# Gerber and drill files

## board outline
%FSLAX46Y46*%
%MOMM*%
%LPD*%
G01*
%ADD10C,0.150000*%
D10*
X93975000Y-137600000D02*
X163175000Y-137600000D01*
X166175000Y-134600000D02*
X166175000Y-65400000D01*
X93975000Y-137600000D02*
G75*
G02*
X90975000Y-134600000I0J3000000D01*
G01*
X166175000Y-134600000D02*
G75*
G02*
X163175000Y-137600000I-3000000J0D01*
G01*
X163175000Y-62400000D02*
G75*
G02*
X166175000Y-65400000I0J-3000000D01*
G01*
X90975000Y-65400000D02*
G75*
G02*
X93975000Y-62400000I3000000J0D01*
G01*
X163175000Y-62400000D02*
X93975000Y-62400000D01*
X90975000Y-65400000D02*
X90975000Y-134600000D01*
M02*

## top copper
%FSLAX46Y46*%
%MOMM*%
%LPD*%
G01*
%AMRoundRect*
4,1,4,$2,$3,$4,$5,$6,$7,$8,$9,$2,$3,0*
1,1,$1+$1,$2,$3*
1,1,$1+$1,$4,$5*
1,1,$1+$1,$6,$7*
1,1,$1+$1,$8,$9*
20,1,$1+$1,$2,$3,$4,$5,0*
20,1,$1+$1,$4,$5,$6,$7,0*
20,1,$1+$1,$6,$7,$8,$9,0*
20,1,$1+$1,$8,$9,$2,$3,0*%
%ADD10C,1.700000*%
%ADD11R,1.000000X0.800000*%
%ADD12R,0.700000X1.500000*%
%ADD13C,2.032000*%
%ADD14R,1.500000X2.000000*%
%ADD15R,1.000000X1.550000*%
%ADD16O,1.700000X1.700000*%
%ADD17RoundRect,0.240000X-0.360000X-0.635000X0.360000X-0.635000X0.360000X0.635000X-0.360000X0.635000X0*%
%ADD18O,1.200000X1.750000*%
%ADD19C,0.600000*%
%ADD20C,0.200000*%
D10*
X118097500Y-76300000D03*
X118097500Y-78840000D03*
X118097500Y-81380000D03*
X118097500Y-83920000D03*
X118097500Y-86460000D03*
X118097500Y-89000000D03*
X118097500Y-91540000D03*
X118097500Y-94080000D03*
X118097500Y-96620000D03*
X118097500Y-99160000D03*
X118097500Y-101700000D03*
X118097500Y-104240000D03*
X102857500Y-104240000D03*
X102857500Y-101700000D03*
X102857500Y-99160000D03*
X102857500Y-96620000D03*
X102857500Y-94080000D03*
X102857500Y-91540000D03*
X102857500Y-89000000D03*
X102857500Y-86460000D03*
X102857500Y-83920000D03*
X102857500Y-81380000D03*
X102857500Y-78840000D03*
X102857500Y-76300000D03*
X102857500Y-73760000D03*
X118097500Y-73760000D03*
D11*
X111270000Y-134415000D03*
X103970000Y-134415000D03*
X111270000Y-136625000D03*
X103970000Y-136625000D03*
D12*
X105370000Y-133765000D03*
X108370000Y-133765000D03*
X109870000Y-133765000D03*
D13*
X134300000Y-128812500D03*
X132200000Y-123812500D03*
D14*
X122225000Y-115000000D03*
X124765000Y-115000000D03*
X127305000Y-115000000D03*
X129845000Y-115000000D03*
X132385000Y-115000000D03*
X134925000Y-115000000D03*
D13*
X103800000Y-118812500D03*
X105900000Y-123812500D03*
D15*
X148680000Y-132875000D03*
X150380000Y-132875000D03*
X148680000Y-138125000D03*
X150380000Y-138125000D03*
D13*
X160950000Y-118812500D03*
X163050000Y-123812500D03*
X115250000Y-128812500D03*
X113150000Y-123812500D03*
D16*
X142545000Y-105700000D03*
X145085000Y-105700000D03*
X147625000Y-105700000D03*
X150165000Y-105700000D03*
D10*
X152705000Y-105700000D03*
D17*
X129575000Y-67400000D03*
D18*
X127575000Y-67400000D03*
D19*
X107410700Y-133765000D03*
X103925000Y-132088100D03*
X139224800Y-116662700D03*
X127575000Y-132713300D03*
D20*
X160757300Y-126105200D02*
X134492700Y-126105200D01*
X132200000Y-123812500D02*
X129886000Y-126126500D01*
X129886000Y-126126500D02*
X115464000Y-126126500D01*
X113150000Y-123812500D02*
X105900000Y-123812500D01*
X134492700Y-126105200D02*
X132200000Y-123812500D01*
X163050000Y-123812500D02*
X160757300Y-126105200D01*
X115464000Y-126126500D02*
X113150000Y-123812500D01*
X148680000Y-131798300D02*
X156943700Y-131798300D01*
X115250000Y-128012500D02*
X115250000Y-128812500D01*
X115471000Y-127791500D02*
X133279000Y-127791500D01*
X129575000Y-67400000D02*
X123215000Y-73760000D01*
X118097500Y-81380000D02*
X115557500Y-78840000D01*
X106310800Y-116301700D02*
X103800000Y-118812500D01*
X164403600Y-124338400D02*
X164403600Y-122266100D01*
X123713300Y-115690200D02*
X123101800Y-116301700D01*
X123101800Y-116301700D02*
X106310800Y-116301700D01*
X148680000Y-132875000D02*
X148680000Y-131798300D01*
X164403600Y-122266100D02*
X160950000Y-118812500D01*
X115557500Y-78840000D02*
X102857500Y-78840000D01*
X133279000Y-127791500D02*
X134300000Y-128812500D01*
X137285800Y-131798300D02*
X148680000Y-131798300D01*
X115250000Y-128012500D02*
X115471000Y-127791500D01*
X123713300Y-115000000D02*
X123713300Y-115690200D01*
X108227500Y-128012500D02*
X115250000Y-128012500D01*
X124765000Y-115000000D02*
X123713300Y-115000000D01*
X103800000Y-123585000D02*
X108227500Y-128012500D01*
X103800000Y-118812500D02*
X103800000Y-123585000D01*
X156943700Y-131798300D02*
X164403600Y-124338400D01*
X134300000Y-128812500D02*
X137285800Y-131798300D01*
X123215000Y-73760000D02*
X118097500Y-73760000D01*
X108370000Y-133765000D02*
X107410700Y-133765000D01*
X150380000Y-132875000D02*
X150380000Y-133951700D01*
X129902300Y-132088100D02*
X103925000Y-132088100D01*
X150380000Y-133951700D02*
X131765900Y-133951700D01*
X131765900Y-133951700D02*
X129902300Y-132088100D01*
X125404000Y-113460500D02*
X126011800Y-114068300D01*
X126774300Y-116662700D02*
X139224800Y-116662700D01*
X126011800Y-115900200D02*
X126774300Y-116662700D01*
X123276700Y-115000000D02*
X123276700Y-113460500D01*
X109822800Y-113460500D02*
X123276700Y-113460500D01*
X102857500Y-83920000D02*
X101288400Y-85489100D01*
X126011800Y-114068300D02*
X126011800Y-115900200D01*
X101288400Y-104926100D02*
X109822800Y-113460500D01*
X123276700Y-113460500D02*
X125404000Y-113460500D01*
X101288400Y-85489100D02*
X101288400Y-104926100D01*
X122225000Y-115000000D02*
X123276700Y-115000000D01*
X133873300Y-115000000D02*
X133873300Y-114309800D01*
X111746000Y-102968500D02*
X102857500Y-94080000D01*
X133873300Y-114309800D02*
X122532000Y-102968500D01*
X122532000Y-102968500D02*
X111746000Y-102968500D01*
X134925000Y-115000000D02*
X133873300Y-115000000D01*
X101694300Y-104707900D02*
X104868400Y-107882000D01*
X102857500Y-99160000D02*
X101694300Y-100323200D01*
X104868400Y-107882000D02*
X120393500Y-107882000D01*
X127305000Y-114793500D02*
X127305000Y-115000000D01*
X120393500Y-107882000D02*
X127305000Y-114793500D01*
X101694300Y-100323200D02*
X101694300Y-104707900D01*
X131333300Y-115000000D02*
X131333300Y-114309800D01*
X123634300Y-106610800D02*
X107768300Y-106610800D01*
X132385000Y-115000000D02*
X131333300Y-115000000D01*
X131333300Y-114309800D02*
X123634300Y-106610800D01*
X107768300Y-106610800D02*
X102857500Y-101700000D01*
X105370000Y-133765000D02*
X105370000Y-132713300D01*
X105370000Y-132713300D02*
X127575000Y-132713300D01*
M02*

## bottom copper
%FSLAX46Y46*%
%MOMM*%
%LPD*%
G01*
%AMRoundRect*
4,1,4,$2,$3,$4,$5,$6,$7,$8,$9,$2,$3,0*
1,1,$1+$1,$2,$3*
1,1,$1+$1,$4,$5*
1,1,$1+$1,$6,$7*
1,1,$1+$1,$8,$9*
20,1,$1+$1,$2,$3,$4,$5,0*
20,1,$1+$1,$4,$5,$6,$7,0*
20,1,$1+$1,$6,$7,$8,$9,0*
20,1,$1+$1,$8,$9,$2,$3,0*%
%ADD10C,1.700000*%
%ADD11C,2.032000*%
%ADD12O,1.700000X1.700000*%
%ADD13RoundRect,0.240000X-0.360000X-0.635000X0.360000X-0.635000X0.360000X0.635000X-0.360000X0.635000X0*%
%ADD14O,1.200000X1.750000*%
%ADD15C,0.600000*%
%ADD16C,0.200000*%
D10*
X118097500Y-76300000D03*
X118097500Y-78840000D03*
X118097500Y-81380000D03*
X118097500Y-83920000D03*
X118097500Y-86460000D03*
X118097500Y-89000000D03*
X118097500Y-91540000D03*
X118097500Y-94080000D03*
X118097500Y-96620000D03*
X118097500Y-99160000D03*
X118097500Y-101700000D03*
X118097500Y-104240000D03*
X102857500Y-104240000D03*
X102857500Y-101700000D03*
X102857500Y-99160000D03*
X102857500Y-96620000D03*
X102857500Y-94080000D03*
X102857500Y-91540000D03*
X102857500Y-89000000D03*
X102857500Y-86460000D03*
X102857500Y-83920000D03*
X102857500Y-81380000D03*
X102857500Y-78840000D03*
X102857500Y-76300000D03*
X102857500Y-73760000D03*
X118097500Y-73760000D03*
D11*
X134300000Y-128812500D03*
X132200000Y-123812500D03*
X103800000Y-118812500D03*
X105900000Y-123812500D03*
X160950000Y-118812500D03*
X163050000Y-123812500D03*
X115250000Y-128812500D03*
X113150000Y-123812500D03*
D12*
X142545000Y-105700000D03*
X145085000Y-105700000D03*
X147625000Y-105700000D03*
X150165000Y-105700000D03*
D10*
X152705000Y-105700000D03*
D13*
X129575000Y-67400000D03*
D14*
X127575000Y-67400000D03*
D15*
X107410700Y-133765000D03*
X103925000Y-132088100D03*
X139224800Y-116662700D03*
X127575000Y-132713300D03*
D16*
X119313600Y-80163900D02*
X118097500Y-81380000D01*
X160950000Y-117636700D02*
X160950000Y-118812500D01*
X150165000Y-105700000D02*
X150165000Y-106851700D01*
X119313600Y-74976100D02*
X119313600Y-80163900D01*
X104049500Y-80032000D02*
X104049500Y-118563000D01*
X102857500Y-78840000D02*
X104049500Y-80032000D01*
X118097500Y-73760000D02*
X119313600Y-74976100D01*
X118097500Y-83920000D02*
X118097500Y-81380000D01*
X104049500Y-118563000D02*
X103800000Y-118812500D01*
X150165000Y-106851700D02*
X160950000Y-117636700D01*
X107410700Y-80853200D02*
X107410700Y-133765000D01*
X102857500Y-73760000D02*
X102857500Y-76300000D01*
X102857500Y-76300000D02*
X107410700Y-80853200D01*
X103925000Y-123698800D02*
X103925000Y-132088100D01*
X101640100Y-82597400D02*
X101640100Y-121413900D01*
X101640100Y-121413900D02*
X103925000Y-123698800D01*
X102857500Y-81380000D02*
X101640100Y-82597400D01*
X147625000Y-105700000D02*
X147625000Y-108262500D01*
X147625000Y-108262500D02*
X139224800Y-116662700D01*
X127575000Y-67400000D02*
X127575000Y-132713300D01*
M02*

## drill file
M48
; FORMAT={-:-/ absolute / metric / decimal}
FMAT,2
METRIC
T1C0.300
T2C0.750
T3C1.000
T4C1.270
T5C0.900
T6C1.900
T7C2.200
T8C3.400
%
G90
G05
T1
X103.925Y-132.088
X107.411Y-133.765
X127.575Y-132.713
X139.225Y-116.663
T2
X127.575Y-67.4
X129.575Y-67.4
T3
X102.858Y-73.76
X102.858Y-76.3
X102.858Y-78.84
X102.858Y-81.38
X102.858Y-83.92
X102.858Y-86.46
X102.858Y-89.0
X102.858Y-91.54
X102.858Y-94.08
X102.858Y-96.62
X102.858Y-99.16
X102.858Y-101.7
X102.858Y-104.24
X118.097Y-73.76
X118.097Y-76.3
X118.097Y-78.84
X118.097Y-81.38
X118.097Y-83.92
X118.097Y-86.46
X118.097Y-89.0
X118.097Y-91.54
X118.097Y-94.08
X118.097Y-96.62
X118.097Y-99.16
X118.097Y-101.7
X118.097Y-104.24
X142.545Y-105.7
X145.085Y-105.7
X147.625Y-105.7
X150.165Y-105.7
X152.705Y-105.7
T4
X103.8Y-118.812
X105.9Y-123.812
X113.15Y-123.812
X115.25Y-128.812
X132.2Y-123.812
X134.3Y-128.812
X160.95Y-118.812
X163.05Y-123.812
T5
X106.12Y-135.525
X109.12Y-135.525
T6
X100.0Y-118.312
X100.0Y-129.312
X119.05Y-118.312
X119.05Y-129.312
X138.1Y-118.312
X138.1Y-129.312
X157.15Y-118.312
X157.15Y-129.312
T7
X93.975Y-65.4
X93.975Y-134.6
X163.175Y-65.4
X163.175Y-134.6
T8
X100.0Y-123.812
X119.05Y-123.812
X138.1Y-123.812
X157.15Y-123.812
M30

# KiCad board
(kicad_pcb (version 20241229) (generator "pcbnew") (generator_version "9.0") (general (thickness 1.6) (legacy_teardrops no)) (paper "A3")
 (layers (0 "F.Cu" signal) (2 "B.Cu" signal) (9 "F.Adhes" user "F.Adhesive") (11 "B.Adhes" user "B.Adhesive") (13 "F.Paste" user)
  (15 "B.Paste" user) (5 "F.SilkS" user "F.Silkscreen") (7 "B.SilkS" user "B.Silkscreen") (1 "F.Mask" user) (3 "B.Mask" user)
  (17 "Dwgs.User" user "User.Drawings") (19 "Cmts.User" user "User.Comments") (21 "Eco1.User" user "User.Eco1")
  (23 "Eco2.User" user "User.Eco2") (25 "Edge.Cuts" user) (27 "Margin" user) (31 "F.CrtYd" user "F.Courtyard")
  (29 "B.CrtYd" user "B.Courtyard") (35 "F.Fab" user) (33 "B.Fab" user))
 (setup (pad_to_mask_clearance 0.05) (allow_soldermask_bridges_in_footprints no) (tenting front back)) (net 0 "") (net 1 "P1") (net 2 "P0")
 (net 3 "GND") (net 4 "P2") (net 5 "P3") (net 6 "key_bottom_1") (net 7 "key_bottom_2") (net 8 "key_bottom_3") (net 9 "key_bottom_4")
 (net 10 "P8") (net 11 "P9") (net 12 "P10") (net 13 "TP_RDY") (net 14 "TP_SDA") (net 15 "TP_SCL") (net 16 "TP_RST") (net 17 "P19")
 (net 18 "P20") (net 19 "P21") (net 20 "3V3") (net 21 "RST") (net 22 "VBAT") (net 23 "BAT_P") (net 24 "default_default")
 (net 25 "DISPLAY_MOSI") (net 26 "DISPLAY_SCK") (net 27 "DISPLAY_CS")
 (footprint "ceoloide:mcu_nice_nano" (layer "F.Cu") (at 110.4775 89)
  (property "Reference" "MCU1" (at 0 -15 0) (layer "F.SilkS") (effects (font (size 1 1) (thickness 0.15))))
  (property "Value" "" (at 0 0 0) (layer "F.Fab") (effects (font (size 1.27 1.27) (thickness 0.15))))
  (pad "1" thru_hole circle (at 7.62 -12.7) (size 1.7 1.7) (drill 1) (layers "*.Cu" "*.Mask") (remove_unused_layers no) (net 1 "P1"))
  (pad "2" thru_hole circle (at 7.62 -10.16) (size 1.7 1.7) (drill 1) (layers "*.Cu" "*.Mask") (remove_unused_layers no) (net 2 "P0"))
  (pad "3" thru_hole circle (at 7.62 -7.62) (size 1.7 1.7) (drill 1) (layers "*.Cu" "*.Mask") (remove_unused_layers no) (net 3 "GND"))
  (pad "4" thru_hole circle (at 7.62 -5.08) (size 1.7 1.7) (drill 1) (layers "*.Cu" "*.Mask") (remove_unused_layers no) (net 3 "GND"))
  (pad "5" thru_hole circle (at 7.62 -2.54) (size 1.7 1.7) (drill 1) (layers "*.Cu" "*.Mask") (remove_unused_layers no) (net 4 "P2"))
  (pad "6" thru_hole circle (at 7.62 0) (size 1.7 1.7) (drill 1) (layers "*.Cu" "*.Mask") (remove_unused_layers no) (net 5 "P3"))
  (pad "7" thru_hole circle (at 7.62 2.54) (size 1.7 1.7) (drill 1) (layers "*.Cu" "*.Mask") (remove_unused_layers no)
   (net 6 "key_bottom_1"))
  (pad "8" thru_hole circle (at 7.62 5.08) (size 1.7 1.7) (drill 1) (layers "*.Cu" "*.Mask") (remove_unused_layers no)
   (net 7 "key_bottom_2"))
  (pad "9" thru_hole circle (at 7.62 7.62) (size 1.7 1.7) (drill 1) (layers "*.Cu" "*.Mask") (remove_unused_layers no)
   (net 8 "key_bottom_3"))
  (pad "10" thru_hole circle (at 7.62 10.16) (size 1.7 1.7) (drill 1) (layers "*.Cu" "*.Mask") (remove_unused_layers no)
   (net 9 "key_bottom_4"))
  (pad "11" thru_hole circle (at 7.62 12.7) (size 1.7 1.7) (drill 1) (layers "*.Cu" "*.Mask") (remove_unused_layers no) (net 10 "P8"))
  (pad "12" thru_hole circle (at 7.62 15.24) (size 1.7 1.7) (drill 1) (layers "*.Cu" "*.Mask") (remove_unused_layers no) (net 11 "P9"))
  (pad "13" thru_hole circle (at -7.62 15.24) (size 1.7 1.7) (drill 1) (layers "*.Cu" "*.Mask") (remove_unused_layers no) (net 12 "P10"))
  (pad "14" thru_hole circle (at -7.62 12.7) (size 1.7 1.7) (drill 1) (layers "*.Cu" "*.Mask") (remove_unused_layers no) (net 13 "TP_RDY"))
  (pad "15" thru_hole circle (at -7.62 10.16) (size 1.7 1.7) (drill 1) (layers "*.Cu" "*.Mask") (remove_unused_layers no) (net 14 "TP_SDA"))
  (pad "16" thru_hole circle (at -7.62 7.62) (size 1.7 1.7) (drill 1) (layers "*.Cu" "*.Mask") (remove_unused_layers no) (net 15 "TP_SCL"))
  (pad "17" thru_hole circle (at -7.62 5.08) (size 1.7 1.7) (drill 1) (layers "*.Cu" "*.Mask") (remove_unused_layers no) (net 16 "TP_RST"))
  (pad "18" thru_hole circle (at -7.62 2.54) (size 1.7 1.7) (drill 1) (layers "*.Cu" "*.Mask") (remove_unused_layers no) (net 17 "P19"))
  (pad "19" thru_hole circle (at -7.62 0) (size 1.7 1.7) (drill 1) (layers "*.Cu" "*.Mask") (remove_unused_layers no) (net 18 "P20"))
  (pad "20" thru_hole circle (at -7.62 -2.54) (size 1.7 1.7) (drill 1) (layers "*.Cu" "*.Mask") (remove_unused_layers no) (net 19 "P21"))
  (pad "21" thru_hole circle (at -7.62 -5.08) (size 1.7 1.7) (drill 1) (layers "*.Cu" "*.Mask") (remove_unused_layers no) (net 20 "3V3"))
  (pad "22" thru_hole circle (at -7.62 -7.62) (size 1.7 1.7) (drill 1) (layers "*.Cu" "*.Mask") (remove_unused_layers no) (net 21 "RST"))
  (pad "23" thru_hole circle (at -7.62 -10.16) (size 1.7 1.7) (drill 1) (layers "*.Cu" "*.Mask") (remove_unused_layers no) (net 3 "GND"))
  (pad "24" thru_hole circle (at -7.62 -12.7) (size 1.7 1.7) (drill 1) (layers "*.Cu" "*.Mask") (remove_unused_layers no) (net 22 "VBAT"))
  (pad "25" thru_hole circle (at -7.62 -15.24) (size 1.7 1.7) (drill 1) (layers "*.Cu" "*.Mask") (remove_unused_layers no) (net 22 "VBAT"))
  (pad "26" thru_hole circle (at 7.62 -15.24) (size 1.7 1.7) (drill 1) (layers "*.Cu" "*.Mask") (remove_unused_layers no) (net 3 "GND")))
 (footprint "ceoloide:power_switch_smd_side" (layer "F.Cu") (at 107.62 135.5 -90)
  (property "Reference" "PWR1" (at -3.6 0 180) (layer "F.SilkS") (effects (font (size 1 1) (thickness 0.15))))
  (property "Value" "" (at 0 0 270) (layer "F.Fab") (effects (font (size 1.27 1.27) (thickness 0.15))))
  (pad "" smd rect (at -1.085 -3.65) (size 1 0.8) (layers "F.Cu" "F.Mask" "F.Paste"))
  (pad "" smd rect (at -1.085 3.65) (size 1 0.8) (layers "F.Cu" "F.Mask" "F.Paste"))
  (pad "" np_thru_hole circle (at 0.025 -1.5) (size 0.9 0.9) (drill 0.9) (layers "*.Cu" "*.Mask"))
  (pad "" np_thru_hole circle (at 0.025 1.5) (size 0.9 0.9) (drill 0.9) (layers "*.Cu" "*.Mask"))
  (pad "" smd rect (at 1.125 -3.65) (size 1 0.8) (layers "F.Cu" "F.Mask" "F.Paste"))
  (pad "" smd rect (at 1.125 3.65) (size 1 0.8) (layers "F.Cu" "F.Mask" "F.Paste"))
  (pad "1" smd rect (at -1.735 2.25) (size 0.7 1.5) (layers "F.Cu" "F.Mask" "F.Paste") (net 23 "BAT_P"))
  (pad "2" smd rect (at -1.735 -0.75) (size 0.7 1.5) (layers "F.Cu" "F.Mask" "F.Paste") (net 22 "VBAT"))
  (pad "3" smd rect (at -1.735 -2.25) (size 0.7 1.5) (layers "F.Cu" "F.Mask" "F.Paste")))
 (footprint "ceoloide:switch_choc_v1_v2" (layer "F.Cu") (at 138.1 123.8125 90)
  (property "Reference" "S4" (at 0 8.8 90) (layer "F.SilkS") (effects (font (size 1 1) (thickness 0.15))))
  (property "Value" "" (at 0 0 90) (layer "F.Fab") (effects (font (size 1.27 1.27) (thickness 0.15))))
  (pad "" np_thru_hole circle (at -5.5 0 90) (size 1.9 1.9) (drill 1.9) (layers "*.Cu" "*.Mask"))
  (pad "" np_thru_hole circle (at 0 0 90) (size 3.4 3.4) (drill 3.4) (layers "*.Cu" "*.Mask"))
  (pad "" np_thru_hole circle (at 5.5 0 90) (size 1.9 1.9) (drill 1.9) (layers "*.Cu" "*.Mask"))
  (pad "1" thru_hole circle (at -5 -3.8 285) (size 2.032 2.032) (drill 1.27) (layers "*.Cu" "*.Mask") (remove_unused_layers no)
   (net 3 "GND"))
  (pad "2" thru_hole circle (at 0 -5.9 285) (size 2.032 2.032) (drill 1.27) (layers "*.Cu" "*.Mask") (remove_unused_layers no)
   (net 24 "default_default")))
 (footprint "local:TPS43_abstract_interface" (layer "F.Cu") (at 128.575 91)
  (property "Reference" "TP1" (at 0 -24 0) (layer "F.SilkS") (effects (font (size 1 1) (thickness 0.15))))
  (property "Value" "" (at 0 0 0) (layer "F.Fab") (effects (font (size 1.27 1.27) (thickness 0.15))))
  (pad "1" smd rect (at -6.35 24) (size 1.5 2) (layers "F.Cu" "F.Mask" "F.Paste") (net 20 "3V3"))
  (pad "2" smd rect (at -3.81 24) (size 1.5 2) (layers "F.Cu" "F.Mask" "F.Paste") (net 3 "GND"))
  (pad "3" smd rect (at -1.27 24) (size 1.5 2) (layers "F.Cu" "F.Mask" "F.Paste") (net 14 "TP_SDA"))
  (pad "4" smd rect (at 1.27 24) (size 1.5 2) (layers "F.Cu" "F.Mask" "F.Paste") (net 15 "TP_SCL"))
  (pad "5" smd rect (at 3.81 24) (size 1.5 2) (layers "F.Cu" "F.Mask" "F.Paste") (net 13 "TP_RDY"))
  (pad "6" smd rect (at 6.35 24) (size 1.5 2) (layers "F.Cu" "F.Mask" "F.Paste") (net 16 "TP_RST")))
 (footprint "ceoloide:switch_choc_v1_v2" (layer "F.Cu") (at 100 123.8125 -90)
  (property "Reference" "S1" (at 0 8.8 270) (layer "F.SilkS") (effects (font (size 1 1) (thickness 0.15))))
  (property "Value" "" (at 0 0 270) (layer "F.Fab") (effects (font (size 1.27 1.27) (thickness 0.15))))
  (pad "" np_thru_hole circle (at -5.5 0 270) (size 1.9 1.9) (drill 1.9) (layers "*.Cu" "*.Mask"))
  (pad "" np_thru_hole circle (at 0 0 270) (size 3.4 3.4) (drill 3.4) (layers "*.Cu" "*.Mask"))
  (pad "" np_thru_hole circle (at 5.5 0 270) (size 1.9 1.9) (drill 1.9) (layers "*.Cu" "*.Mask"))
  (pad "1" thru_hole circle (at -5 -3.8 105) (size 2.032 2.032) (drill 1.27) (layers "*.Cu" "*.Mask") (remove_unused_layers no)
   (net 3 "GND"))
  (pad "2" thru_hole circle (at 0 -5.9 105) (size 2.032 2.032) (drill 1.27) (layers "*.Cu" "*.Mask") (remove_unused_layers no)
   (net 24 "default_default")))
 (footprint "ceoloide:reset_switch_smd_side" (layer "F.Cu") (at 149.53 135.5 90)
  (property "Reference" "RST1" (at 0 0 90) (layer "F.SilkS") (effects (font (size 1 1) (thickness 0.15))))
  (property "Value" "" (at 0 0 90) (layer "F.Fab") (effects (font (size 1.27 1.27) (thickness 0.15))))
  (pad "1" smd rect (at 2.625 -0.85 270) (size 1.55 1) (layers "F.Cu" "F.Mask" "F.Paste") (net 3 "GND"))
  (pad "2" smd rect (at 2.625 0.85 270) (size 1.55 1) (layers "F.Cu" "F.Mask" "F.Paste") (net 21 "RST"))
  (pad "3" smd rect (at -2.625 -0.85 270) (size 1.55 1) (layers "F.Cu" "F.Mask" "F.Paste") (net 3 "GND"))
  (pad "4" smd rect (at -2.625 0.85 270) (size 1.55 1) (layers "F.Cu" "F.Mask" "F.Paste") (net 21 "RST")))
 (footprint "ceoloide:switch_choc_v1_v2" (layer "F.Cu") (at 157.15 123.8125 -90)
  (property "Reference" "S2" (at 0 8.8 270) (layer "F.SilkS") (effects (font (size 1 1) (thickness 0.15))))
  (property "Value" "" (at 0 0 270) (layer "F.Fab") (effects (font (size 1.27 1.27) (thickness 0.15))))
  (pad "" np_thru_hole circle (at -5.5 0 270) (size 1.9 1.9) (drill 1.9) (layers "*.Cu" "*.Mask"))
  (pad "" np_thru_hole circle (at 0 0 270) (size 3.4 3.4) (drill 3.4) (layers "*.Cu" "*.Mask"))
  (pad "" np_thru_hole circle (at 5.5 0 270) (size 1.9 1.9) (drill 1.9) (layers "*.Cu" "*.Mask"))
  (pad "1" thru_hole circle (at -5 -3.8 105) (size 2.032 2.032) (drill 1.27) (layers "*.Cu" "*.Mask") (remove_unused_layers no)
   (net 3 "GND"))
  (pad "2" thru_hole circle (at 0 -5.9 105) (size 2.032 2.032) (drill 1.27) (layers "*.Cu" "*.Mask") (remove_unused_layers no)
   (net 24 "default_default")))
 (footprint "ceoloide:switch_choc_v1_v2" (layer "F.Cu") (at 119.05 123.8125 90)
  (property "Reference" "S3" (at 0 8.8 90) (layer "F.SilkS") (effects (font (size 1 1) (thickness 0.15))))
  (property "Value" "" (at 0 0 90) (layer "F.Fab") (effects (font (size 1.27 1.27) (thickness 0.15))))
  (pad "" np_thru_hole circle (at -5.5 0 90) (size 1.9 1.9) (drill 1.9) (layers "*.Cu" "*.Mask"))
  (pad "" np_thru_hole circle (at 0 0 90) (size 3.4 3.4) (drill 3.4) (layers "*.Cu" "*.Mask"))
  (pad "" np_thru_hole circle (at 5.5 0 90) (size 1.9 1.9) (drill 1.9) (layers "*.Cu" "*.Mask"))
  (pad "1" thru_hole circle (at -5 -3.8 285) (size 2.032 2.032) (drill 1.27) (layers "*.Cu" "*.Mask") (remove_unused_layers no)
   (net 3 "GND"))
  (pad "2" thru_hole circle (at 0 -5.9 285) (size 2.032 2.032) (drill 1.27) (layers "*.Cu" "*.Mask") (remove_unused_layers no)
   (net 24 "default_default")))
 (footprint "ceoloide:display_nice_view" (layer "F.Cu") (at 147.625 89)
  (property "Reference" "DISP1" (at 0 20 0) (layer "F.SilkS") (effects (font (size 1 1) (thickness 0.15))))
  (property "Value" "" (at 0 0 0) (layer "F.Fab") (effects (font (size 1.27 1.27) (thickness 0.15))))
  (pad "1" thru_hole oval (at -5.08 16.7 270) (size 1.7 1.7) (drill 1) (layers "*.Cu" "*.Mask") (remove_unused_layers no)
   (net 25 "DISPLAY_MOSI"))
  (pad "2" thru_hole oval (at -2.54 16.7 270) (size 1.7 1.7) (drill 1) (layers "*.Cu" "*.Mask") (remove_unused_layers no)
   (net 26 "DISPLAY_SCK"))
  (pad "3" thru_hole oval (at 0 16.7 270) (size 1.7 1.7) (drill 1) (layers "*.Cu" "*.Mask") (remove_unused_layers no) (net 20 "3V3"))
  (pad "4" thru_hole oval (at 2.54 16.7 270) (size 1.7 1.7) (drill 1) (layers "*.Cu" "*.Mask") (remove_unused_layers no) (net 3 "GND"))
  (pad "5" thru_hole circle (at 5.08 16.7 270) (size 1.7 1.7) (drill 1) (layers "*.Cu" "*.Mask") (remove_unused_layers no)
   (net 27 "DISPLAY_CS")))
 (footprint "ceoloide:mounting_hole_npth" (layer "B.Cu") (at 93.975 134.6)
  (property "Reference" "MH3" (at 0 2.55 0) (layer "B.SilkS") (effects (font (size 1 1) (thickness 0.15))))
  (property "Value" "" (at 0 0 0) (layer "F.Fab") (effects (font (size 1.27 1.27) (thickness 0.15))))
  (pad "" np_thru_hole circle (at 0 0) (size 2.2 2.2) (drill 2.2) (layers "*.Cu" "*.Mask")))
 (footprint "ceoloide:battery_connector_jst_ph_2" (layer "B.Cu") (at 128.575 67.4)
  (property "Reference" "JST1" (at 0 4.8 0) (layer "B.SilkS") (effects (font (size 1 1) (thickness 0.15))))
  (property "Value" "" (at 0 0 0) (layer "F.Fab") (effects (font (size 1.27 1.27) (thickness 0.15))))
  (pad "1" thru_hole roundrect (at 1 0) (size 1.2 1.75) (drill 0.75) (layers "*.Cu" "*.Mask") (remove_unused_layers no)
   (roundrect_rratio 0.2) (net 3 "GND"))
  (pad "2" thru_hole oval (at -1 0) (size 1.2 1.75) (drill 0.75) (layers "*.Cu" "*.Mask") (remove_unused_layers no) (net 23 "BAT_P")))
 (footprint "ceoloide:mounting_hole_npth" (layer "B.Cu") (at 163.175 134.6)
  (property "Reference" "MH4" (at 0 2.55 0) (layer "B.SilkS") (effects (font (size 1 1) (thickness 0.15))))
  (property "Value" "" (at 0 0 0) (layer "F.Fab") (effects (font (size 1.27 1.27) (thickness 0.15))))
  (pad "" np_thru_hole circle (at 0 0) (size 2.2 2.2) (drill 2.2) (layers "*.Cu" "*.Mask")))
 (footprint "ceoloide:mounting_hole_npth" (layer "B.Cu") (at 163.175 65.4)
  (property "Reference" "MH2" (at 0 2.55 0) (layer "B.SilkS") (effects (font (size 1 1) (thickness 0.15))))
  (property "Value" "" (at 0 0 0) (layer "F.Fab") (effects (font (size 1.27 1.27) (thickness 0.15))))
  (pad "" np_thru_hole circle (at 0 0) (size 2.2 2.2) (drill 2.2) (layers "*.Cu" "*.Mask")))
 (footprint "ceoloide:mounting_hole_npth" (layer "B.Cu") (at 93.975 65.4)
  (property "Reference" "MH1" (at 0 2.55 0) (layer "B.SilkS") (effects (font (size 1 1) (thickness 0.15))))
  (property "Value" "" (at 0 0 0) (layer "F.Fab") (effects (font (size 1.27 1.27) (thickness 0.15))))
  (pad "" np_thru_hole circle (at 0 0) (size 2.2 2.2) (drill 2.2) (layers "*.Cu" "*.Mask")))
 (gr_line (start 93.975 137.6) (end 163.175 137.6) (stroke (width 0.15) (type default)) (layer "Edge.Cuts"))
 (gr_line (start 166.175 134.6) (end 166.175 65.4) (stroke (width 0.15) (type default)) (layer "Edge.Cuts"))
 (gr_arc (start 93.975 137.6) (mid 91.85368 136.72132) (end 90.975 134.6) (stroke (width 0.15) (type default)) (layer "Edge.Cuts"))
 (gr_arc (start 166.175 134.6) (mid 165.29632 136.72132) (end 163.175 137.6) (stroke (width 0.15) (type default)) (layer "Edge.Cuts"))
 (gr_arc (start 163.175 62.4) (mid 165.29632 63.27868) (end 166.175 65.4) (stroke (width 0.15) (type default)) (layer "Edge.Cuts"))
 (gr_arc (start 90.975 65.4) (mid 91.85368 63.27868) (end 93.975 62.4) (stroke (width 0.15) (type default)) (layer "Edge.Cuts"))
 (gr_line (start 163.175 62.4) (end 93.975 62.4) (stroke (width 0.15) (type default)) (layer "Edge.Cuts"))
 (gr_line (start 90.975 65.4) (end 90.975 134.6) (stroke (width 0.15) (type default)) (layer "Edge.Cuts"))
 (segment (start 160.7573 126.1052) (end 134.4927 126.1052) (width 0.2) (layer "F.Cu") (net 24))
 (segment (start 132.2 123.8125) (end 129.886 126.1265) (width 0.2) (layer "F.Cu") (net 24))
 (segment (start 129.886 126.1265) (end 115.464 126.1265) (width 0.2) (layer "F.Cu") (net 24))
 (segment (start 113.15 123.8125) (end 105.9 123.8125) (width 0.2) (layer "F.Cu") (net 24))
 (segment (start 134.4927 126.1052) (end 132.2 123.8125) (width 0.2) (layer "F.Cu") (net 24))
 (segment (start 163.05 123.8125) (end 160.7573 126.1052) (width 0.2) (layer "F.Cu") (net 24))
 (segment (start 115.464 126.1265) (end 113.15 123.8125) (width 0.2) (layer "F.Cu") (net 24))
 (segment (start 148.68 131.7983) (end 156.9437 131.7983) (width 0.2) (layer "F.Cu") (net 3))
 (segment (start 115.25 128.0125) (end 115.25 128.8125) (width 0.2) (layer "F.Cu") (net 3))
 (segment (start 115.471 127.7915) (end 133.279 127.7915) (width 0.2) (layer "F.Cu") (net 3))
 (segment (start 129.575 67.4) (end 123.215 73.76) (width 0.2) (layer "F.Cu") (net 3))
 (segment (start 118.0975 81.38) (end 115.5575 78.84) (width 0.2) (layer "F.Cu") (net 3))
 (segment (start 106.3108 116.3017) (end 103.8 118.8125) (width 0.2) (layer "F.Cu") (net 3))
 (segment (start 164.4036 124.3384) (end 164.4036 122.2661) (width 0.2) (layer "F.Cu") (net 3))
 (segment (start 123.7133 115.6902) (end 123.1018 116.3017) (width 0.2) (layer "F.Cu") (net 3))
 (segment (start 123.1018 116.3017) (end 106.3108 116.3017) (width 0.2) (layer "F.Cu") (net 3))
 (segment (start 148.68 132.875) (end 148.68 131.7983) (width 0.2) (layer "F.Cu") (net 3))
 (segment (start 164.4036 122.2661) (end 160.95 118.8125) (width 0.2) (layer "F.Cu") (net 3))
 (segment (start 115.5575 78.84) (end 102.8575 78.84) (width 0.2) (layer "F.Cu") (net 3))
 (segment (start 133.279 127.7915) (end 134.3 128.8125) (width 0.2) (layer "F.Cu") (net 3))
 (segment (start 137.2858 131.7983) (end 148.68 131.7983) (width 0.2) (layer "F.Cu") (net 3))
 (segment (start 115.25 128.0125) (end 115.471 127.7915) (width 0.2) (layer "F.Cu") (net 3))
 (segment (start 123.7133 115) (end 123.7133 115.6902) (width 0.2) (layer "F.Cu") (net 3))
 (segment (start 108.2275 128.0125) (end 115.25 128.0125) (width 0.2) (layer "F.Cu") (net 3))
 (segment (start 124.765 115) (end 123.7133 115) (width 0.2) (layer "F.Cu") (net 3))
 (segment (start 103.8 123.585) (end 108.2275 128.0125) (width 0.2) (layer "F.Cu") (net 3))
 (segment (start 103.8 118.8125) (end 103.8 123.585) (width 0.2) (layer "F.Cu") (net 3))
 (segment (start 156.9437 131.7983) (end 164.4036 124.3384) (width 0.2) (layer "F.Cu") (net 3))
 (segment (start 134.3 128.8125) (end 137.2858 131.7983) (width 0.2) (layer "F.Cu") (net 3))
 (segment (start 123.215 73.76) (end 118.0975 73.76) (width 0.2) (layer "F.Cu") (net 3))
 (segment (start 119.3136 80.1639) (end 118.0975 81.38) (width 0.2) (layer "B.Cu") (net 3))
 (segment (start 160.95 117.6367) (end 160.95 118.8125) (width 0.2) (layer "B.Cu") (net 3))
 (segment (start 150.165 105.7) (end 150.165 106.8517) (width 0.2) (layer "B.Cu") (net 3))
 (segment (start 119.3136 74.9761) (end 119.3136 80.1639) (width 0.2) (layer "B.Cu") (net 3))
 (segment (start 104.0495 80.032) (end 104.0495 118.563) (width 0.2) (layer "B.Cu") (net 3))
 (segment (start 102.8575 78.84) (end 104.0495 80.032) (width 0.2) (layer "B.Cu") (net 3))
 (segment (start 118.0975 73.76) (end 119.3136 74.9761) (width 0.2) (layer "B.Cu") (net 3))
 (segment (start 118.0975 83.92) (end 118.0975 81.38) (width 0.2) (layer "B.Cu") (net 3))
 (segment (start 104.0495 118.563) (end 103.8 118.8125) (width 0.2) (layer "B.Cu") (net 3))
 (segment (start 150.165 106.8517) (end 160.95 117.6367) (width 0.2) (layer "B.Cu") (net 3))
 (segment (start 108.37 133.765) (end 107.4107 133.765) (width 0.2) (layer "F.Cu") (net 22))
 (via (at 107.4107 133.765) (size 0.6) (drill 0.3) (layers "F.Cu" "B.Cu") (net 22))
 (segment (start 107.4107 80.8532) (end 107.4107 133.765) (width 0.2) (layer "B.Cu") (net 22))
 (segment (start 102.8575 73.76) (end 102.8575 76.3) (width 0.2) (layer "B.Cu") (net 22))
 (segment (start 102.8575 76.3) (end 107.4107 80.8532) (width 0.2) (layer "B.Cu") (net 22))
 (segment (start 150.38 132.875) (end 150.38 133.9517) (width 0.2) (layer "F.Cu") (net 21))
 (segment (start 129.9023 132.0881) (end 103.925 132.0881) (width 0.2) (layer "F.Cu") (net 21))
 (segment (start 150.38 133.9517) (end 131.7659 133.9517) (width 0.2) (layer "F.Cu") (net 21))
 (segment (start 131.7659 133.9517) (end 129.9023 132.0881) (width 0.2) (layer "F.Cu") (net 21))
 (via (at 103.925 132.0881) (size 0.6) (drill 0.3) (layers "F.Cu" "B.Cu") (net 21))
 (segment (start 103.925 123.6988) (end 103.925 132.0881) (width 0.2) (layer "B.Cu") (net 21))
 (segment (start 101.6401 82.5974) (end 101.6401 121.4139) (width 0.2) (layer "B.Cu") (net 21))
 (segment (start 101.6401 121.4139) (end 103.925 123.6988) (width 0.2) (layer "B.Cu") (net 21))
 (segment (start 102.8575 81.38) (end 101.6401 82.5974) (width 0.2) (layer "B.Cu") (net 21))
 (segment (start 125.404 113.4605) (end 126.0118 114.0683) (width 0.2) (layer "F.Cu") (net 20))
 (segment (start 126.7743 116.6627) (end 139.2248 116.6627) (width 0.2) (layer "F.Cu") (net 20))
 (segment (start 126.0118 115.9002) (end 126.7743 116.6627) (width 0.2) (layer "F.Cu") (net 20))
 (segment (start 123.2767 115) (end 123.2767 113.4605) (width 0.2) (layer "F.Cu") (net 20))
 (segment (start 109.8228 113.4605) (end 123.2767 113.4605) (width 0.2) (layer "F.Cu") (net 20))
 (segment (start 102.8575 83.92) (end 101.2884 85.4891) (width 0.2) (layer "F.Cu") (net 20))
 (segment (start 126.0118 114.0683) (end 126.0118 115.9002) (width 0.2) (layer "F.Cu") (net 20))
 (segment (start 101.2884 104.9261) (end 109.8228 113.4605) (width 0.2) (layer "F.Cu") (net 20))
 (segment (start 123.2767 113.4605) (end 125.404 113.4605) (width 0.2) (layer "F.Cu") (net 20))
 (segment (start 101.2884 85.4891) (end 101.2884 104.9261) (width 0.2) (layer "F.Cu") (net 20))
 (segment (start 122.225 115) (end 123.2767 115) (width 0.2) (layer "F.Cu") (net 20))
 (via (at 139.2248 116.6627) (size 0.6) (drill 0.3) (layers "F.Cu" "B.Cu") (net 20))
 (segment (start 147.625 105.7) (end 147.625 108.2625) (width 0.2) (layer "B.Cu") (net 20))
 (segment (start 147.625 108.2625) (end 139.2248 116.6627) (width 0.2) (layer "B.Cu") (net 20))
 (segment (start 133.8733 115) (end 133.8733 114.3098) (width 0.2) (layer "F.Cu") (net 16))
 (segment (start 111.746 102.9685) (end 102.8575 94.08) (width 0.2) (layer "F.Cu") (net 16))
 (segment (start 133.8733 114.3098) (end 122.532 102.9685) (width 0.2) (layer "F.Cu") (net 16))
 (segment (start 122.532 102.9685) (end 111.746 102.9685) (width 0.2) (layer "F.Cu") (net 16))
 (segment (start 134.925 115) (end 133.8733 115) (width 0.2) (layer "F.Cu") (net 16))
 (segment (start 101.6943 104.7079) (end 104.8684 107.882) (width 0.2) (layer "F.Cu") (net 14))
 (segment (start 102.8575 99.16) (end 101.6943 100.3232) (width 0.2) (layer "F.Cu") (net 14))
 (segment (start 104.8684 107.882) (end 120.3935 107.882) (width 0.2) (layer "F.Cu") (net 14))
 (segment (start 127.305 114.7935) (end 127.305 115) (width 0.2) (layer "F.Cu") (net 14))
 (segment (start 120.3935 107.882) (end 127.305 114.7935) (width 0.2) (layer "F.Cu") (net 14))
 (segment (start 101.6943 100.3232) (end 101.6943 104.7079) (width 0.2) (layer "F.Cu") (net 14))
 (segment (start 131.3333 115) (end 131.3333 114.3098) (width 0.2) (layer "F.Cu") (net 13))
 (segment (start 123.6343 106.6108) (end 107.7683 106.6108) (width 0.2) (layer "F.Cu") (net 13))
 (segment (start 132.385 115) (end 131.3333 115) (width 0.2) (layer "F.Cu") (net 13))
 (segment (start 131.3333 114.3098) (end 123.6343 106.6108) (width 0.2) (layer "F.Cu") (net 13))
 (segment (start 107.7683 106.6108) (end 102.8575 101.7) (width 0.2) (layer "F.Cu") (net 13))
 (segment (start 105.37 133.765) (end 105.37 132.7133) (width 0.2) (layer "F.Cu") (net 23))
 (segment (start 105.37 132.7133) (end 127.575 132.7133) (width 0.2) (layer "F.Cu") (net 23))
 (via (at 127.575 132.7133) (size 0.6) (drill 0.3) (layers "F.Cu" "B.Cu") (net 23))
 (segment (start 127.575 67.4) (end 127.575 132.7133) (width 0.2) (layer "B.Cu") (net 23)))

